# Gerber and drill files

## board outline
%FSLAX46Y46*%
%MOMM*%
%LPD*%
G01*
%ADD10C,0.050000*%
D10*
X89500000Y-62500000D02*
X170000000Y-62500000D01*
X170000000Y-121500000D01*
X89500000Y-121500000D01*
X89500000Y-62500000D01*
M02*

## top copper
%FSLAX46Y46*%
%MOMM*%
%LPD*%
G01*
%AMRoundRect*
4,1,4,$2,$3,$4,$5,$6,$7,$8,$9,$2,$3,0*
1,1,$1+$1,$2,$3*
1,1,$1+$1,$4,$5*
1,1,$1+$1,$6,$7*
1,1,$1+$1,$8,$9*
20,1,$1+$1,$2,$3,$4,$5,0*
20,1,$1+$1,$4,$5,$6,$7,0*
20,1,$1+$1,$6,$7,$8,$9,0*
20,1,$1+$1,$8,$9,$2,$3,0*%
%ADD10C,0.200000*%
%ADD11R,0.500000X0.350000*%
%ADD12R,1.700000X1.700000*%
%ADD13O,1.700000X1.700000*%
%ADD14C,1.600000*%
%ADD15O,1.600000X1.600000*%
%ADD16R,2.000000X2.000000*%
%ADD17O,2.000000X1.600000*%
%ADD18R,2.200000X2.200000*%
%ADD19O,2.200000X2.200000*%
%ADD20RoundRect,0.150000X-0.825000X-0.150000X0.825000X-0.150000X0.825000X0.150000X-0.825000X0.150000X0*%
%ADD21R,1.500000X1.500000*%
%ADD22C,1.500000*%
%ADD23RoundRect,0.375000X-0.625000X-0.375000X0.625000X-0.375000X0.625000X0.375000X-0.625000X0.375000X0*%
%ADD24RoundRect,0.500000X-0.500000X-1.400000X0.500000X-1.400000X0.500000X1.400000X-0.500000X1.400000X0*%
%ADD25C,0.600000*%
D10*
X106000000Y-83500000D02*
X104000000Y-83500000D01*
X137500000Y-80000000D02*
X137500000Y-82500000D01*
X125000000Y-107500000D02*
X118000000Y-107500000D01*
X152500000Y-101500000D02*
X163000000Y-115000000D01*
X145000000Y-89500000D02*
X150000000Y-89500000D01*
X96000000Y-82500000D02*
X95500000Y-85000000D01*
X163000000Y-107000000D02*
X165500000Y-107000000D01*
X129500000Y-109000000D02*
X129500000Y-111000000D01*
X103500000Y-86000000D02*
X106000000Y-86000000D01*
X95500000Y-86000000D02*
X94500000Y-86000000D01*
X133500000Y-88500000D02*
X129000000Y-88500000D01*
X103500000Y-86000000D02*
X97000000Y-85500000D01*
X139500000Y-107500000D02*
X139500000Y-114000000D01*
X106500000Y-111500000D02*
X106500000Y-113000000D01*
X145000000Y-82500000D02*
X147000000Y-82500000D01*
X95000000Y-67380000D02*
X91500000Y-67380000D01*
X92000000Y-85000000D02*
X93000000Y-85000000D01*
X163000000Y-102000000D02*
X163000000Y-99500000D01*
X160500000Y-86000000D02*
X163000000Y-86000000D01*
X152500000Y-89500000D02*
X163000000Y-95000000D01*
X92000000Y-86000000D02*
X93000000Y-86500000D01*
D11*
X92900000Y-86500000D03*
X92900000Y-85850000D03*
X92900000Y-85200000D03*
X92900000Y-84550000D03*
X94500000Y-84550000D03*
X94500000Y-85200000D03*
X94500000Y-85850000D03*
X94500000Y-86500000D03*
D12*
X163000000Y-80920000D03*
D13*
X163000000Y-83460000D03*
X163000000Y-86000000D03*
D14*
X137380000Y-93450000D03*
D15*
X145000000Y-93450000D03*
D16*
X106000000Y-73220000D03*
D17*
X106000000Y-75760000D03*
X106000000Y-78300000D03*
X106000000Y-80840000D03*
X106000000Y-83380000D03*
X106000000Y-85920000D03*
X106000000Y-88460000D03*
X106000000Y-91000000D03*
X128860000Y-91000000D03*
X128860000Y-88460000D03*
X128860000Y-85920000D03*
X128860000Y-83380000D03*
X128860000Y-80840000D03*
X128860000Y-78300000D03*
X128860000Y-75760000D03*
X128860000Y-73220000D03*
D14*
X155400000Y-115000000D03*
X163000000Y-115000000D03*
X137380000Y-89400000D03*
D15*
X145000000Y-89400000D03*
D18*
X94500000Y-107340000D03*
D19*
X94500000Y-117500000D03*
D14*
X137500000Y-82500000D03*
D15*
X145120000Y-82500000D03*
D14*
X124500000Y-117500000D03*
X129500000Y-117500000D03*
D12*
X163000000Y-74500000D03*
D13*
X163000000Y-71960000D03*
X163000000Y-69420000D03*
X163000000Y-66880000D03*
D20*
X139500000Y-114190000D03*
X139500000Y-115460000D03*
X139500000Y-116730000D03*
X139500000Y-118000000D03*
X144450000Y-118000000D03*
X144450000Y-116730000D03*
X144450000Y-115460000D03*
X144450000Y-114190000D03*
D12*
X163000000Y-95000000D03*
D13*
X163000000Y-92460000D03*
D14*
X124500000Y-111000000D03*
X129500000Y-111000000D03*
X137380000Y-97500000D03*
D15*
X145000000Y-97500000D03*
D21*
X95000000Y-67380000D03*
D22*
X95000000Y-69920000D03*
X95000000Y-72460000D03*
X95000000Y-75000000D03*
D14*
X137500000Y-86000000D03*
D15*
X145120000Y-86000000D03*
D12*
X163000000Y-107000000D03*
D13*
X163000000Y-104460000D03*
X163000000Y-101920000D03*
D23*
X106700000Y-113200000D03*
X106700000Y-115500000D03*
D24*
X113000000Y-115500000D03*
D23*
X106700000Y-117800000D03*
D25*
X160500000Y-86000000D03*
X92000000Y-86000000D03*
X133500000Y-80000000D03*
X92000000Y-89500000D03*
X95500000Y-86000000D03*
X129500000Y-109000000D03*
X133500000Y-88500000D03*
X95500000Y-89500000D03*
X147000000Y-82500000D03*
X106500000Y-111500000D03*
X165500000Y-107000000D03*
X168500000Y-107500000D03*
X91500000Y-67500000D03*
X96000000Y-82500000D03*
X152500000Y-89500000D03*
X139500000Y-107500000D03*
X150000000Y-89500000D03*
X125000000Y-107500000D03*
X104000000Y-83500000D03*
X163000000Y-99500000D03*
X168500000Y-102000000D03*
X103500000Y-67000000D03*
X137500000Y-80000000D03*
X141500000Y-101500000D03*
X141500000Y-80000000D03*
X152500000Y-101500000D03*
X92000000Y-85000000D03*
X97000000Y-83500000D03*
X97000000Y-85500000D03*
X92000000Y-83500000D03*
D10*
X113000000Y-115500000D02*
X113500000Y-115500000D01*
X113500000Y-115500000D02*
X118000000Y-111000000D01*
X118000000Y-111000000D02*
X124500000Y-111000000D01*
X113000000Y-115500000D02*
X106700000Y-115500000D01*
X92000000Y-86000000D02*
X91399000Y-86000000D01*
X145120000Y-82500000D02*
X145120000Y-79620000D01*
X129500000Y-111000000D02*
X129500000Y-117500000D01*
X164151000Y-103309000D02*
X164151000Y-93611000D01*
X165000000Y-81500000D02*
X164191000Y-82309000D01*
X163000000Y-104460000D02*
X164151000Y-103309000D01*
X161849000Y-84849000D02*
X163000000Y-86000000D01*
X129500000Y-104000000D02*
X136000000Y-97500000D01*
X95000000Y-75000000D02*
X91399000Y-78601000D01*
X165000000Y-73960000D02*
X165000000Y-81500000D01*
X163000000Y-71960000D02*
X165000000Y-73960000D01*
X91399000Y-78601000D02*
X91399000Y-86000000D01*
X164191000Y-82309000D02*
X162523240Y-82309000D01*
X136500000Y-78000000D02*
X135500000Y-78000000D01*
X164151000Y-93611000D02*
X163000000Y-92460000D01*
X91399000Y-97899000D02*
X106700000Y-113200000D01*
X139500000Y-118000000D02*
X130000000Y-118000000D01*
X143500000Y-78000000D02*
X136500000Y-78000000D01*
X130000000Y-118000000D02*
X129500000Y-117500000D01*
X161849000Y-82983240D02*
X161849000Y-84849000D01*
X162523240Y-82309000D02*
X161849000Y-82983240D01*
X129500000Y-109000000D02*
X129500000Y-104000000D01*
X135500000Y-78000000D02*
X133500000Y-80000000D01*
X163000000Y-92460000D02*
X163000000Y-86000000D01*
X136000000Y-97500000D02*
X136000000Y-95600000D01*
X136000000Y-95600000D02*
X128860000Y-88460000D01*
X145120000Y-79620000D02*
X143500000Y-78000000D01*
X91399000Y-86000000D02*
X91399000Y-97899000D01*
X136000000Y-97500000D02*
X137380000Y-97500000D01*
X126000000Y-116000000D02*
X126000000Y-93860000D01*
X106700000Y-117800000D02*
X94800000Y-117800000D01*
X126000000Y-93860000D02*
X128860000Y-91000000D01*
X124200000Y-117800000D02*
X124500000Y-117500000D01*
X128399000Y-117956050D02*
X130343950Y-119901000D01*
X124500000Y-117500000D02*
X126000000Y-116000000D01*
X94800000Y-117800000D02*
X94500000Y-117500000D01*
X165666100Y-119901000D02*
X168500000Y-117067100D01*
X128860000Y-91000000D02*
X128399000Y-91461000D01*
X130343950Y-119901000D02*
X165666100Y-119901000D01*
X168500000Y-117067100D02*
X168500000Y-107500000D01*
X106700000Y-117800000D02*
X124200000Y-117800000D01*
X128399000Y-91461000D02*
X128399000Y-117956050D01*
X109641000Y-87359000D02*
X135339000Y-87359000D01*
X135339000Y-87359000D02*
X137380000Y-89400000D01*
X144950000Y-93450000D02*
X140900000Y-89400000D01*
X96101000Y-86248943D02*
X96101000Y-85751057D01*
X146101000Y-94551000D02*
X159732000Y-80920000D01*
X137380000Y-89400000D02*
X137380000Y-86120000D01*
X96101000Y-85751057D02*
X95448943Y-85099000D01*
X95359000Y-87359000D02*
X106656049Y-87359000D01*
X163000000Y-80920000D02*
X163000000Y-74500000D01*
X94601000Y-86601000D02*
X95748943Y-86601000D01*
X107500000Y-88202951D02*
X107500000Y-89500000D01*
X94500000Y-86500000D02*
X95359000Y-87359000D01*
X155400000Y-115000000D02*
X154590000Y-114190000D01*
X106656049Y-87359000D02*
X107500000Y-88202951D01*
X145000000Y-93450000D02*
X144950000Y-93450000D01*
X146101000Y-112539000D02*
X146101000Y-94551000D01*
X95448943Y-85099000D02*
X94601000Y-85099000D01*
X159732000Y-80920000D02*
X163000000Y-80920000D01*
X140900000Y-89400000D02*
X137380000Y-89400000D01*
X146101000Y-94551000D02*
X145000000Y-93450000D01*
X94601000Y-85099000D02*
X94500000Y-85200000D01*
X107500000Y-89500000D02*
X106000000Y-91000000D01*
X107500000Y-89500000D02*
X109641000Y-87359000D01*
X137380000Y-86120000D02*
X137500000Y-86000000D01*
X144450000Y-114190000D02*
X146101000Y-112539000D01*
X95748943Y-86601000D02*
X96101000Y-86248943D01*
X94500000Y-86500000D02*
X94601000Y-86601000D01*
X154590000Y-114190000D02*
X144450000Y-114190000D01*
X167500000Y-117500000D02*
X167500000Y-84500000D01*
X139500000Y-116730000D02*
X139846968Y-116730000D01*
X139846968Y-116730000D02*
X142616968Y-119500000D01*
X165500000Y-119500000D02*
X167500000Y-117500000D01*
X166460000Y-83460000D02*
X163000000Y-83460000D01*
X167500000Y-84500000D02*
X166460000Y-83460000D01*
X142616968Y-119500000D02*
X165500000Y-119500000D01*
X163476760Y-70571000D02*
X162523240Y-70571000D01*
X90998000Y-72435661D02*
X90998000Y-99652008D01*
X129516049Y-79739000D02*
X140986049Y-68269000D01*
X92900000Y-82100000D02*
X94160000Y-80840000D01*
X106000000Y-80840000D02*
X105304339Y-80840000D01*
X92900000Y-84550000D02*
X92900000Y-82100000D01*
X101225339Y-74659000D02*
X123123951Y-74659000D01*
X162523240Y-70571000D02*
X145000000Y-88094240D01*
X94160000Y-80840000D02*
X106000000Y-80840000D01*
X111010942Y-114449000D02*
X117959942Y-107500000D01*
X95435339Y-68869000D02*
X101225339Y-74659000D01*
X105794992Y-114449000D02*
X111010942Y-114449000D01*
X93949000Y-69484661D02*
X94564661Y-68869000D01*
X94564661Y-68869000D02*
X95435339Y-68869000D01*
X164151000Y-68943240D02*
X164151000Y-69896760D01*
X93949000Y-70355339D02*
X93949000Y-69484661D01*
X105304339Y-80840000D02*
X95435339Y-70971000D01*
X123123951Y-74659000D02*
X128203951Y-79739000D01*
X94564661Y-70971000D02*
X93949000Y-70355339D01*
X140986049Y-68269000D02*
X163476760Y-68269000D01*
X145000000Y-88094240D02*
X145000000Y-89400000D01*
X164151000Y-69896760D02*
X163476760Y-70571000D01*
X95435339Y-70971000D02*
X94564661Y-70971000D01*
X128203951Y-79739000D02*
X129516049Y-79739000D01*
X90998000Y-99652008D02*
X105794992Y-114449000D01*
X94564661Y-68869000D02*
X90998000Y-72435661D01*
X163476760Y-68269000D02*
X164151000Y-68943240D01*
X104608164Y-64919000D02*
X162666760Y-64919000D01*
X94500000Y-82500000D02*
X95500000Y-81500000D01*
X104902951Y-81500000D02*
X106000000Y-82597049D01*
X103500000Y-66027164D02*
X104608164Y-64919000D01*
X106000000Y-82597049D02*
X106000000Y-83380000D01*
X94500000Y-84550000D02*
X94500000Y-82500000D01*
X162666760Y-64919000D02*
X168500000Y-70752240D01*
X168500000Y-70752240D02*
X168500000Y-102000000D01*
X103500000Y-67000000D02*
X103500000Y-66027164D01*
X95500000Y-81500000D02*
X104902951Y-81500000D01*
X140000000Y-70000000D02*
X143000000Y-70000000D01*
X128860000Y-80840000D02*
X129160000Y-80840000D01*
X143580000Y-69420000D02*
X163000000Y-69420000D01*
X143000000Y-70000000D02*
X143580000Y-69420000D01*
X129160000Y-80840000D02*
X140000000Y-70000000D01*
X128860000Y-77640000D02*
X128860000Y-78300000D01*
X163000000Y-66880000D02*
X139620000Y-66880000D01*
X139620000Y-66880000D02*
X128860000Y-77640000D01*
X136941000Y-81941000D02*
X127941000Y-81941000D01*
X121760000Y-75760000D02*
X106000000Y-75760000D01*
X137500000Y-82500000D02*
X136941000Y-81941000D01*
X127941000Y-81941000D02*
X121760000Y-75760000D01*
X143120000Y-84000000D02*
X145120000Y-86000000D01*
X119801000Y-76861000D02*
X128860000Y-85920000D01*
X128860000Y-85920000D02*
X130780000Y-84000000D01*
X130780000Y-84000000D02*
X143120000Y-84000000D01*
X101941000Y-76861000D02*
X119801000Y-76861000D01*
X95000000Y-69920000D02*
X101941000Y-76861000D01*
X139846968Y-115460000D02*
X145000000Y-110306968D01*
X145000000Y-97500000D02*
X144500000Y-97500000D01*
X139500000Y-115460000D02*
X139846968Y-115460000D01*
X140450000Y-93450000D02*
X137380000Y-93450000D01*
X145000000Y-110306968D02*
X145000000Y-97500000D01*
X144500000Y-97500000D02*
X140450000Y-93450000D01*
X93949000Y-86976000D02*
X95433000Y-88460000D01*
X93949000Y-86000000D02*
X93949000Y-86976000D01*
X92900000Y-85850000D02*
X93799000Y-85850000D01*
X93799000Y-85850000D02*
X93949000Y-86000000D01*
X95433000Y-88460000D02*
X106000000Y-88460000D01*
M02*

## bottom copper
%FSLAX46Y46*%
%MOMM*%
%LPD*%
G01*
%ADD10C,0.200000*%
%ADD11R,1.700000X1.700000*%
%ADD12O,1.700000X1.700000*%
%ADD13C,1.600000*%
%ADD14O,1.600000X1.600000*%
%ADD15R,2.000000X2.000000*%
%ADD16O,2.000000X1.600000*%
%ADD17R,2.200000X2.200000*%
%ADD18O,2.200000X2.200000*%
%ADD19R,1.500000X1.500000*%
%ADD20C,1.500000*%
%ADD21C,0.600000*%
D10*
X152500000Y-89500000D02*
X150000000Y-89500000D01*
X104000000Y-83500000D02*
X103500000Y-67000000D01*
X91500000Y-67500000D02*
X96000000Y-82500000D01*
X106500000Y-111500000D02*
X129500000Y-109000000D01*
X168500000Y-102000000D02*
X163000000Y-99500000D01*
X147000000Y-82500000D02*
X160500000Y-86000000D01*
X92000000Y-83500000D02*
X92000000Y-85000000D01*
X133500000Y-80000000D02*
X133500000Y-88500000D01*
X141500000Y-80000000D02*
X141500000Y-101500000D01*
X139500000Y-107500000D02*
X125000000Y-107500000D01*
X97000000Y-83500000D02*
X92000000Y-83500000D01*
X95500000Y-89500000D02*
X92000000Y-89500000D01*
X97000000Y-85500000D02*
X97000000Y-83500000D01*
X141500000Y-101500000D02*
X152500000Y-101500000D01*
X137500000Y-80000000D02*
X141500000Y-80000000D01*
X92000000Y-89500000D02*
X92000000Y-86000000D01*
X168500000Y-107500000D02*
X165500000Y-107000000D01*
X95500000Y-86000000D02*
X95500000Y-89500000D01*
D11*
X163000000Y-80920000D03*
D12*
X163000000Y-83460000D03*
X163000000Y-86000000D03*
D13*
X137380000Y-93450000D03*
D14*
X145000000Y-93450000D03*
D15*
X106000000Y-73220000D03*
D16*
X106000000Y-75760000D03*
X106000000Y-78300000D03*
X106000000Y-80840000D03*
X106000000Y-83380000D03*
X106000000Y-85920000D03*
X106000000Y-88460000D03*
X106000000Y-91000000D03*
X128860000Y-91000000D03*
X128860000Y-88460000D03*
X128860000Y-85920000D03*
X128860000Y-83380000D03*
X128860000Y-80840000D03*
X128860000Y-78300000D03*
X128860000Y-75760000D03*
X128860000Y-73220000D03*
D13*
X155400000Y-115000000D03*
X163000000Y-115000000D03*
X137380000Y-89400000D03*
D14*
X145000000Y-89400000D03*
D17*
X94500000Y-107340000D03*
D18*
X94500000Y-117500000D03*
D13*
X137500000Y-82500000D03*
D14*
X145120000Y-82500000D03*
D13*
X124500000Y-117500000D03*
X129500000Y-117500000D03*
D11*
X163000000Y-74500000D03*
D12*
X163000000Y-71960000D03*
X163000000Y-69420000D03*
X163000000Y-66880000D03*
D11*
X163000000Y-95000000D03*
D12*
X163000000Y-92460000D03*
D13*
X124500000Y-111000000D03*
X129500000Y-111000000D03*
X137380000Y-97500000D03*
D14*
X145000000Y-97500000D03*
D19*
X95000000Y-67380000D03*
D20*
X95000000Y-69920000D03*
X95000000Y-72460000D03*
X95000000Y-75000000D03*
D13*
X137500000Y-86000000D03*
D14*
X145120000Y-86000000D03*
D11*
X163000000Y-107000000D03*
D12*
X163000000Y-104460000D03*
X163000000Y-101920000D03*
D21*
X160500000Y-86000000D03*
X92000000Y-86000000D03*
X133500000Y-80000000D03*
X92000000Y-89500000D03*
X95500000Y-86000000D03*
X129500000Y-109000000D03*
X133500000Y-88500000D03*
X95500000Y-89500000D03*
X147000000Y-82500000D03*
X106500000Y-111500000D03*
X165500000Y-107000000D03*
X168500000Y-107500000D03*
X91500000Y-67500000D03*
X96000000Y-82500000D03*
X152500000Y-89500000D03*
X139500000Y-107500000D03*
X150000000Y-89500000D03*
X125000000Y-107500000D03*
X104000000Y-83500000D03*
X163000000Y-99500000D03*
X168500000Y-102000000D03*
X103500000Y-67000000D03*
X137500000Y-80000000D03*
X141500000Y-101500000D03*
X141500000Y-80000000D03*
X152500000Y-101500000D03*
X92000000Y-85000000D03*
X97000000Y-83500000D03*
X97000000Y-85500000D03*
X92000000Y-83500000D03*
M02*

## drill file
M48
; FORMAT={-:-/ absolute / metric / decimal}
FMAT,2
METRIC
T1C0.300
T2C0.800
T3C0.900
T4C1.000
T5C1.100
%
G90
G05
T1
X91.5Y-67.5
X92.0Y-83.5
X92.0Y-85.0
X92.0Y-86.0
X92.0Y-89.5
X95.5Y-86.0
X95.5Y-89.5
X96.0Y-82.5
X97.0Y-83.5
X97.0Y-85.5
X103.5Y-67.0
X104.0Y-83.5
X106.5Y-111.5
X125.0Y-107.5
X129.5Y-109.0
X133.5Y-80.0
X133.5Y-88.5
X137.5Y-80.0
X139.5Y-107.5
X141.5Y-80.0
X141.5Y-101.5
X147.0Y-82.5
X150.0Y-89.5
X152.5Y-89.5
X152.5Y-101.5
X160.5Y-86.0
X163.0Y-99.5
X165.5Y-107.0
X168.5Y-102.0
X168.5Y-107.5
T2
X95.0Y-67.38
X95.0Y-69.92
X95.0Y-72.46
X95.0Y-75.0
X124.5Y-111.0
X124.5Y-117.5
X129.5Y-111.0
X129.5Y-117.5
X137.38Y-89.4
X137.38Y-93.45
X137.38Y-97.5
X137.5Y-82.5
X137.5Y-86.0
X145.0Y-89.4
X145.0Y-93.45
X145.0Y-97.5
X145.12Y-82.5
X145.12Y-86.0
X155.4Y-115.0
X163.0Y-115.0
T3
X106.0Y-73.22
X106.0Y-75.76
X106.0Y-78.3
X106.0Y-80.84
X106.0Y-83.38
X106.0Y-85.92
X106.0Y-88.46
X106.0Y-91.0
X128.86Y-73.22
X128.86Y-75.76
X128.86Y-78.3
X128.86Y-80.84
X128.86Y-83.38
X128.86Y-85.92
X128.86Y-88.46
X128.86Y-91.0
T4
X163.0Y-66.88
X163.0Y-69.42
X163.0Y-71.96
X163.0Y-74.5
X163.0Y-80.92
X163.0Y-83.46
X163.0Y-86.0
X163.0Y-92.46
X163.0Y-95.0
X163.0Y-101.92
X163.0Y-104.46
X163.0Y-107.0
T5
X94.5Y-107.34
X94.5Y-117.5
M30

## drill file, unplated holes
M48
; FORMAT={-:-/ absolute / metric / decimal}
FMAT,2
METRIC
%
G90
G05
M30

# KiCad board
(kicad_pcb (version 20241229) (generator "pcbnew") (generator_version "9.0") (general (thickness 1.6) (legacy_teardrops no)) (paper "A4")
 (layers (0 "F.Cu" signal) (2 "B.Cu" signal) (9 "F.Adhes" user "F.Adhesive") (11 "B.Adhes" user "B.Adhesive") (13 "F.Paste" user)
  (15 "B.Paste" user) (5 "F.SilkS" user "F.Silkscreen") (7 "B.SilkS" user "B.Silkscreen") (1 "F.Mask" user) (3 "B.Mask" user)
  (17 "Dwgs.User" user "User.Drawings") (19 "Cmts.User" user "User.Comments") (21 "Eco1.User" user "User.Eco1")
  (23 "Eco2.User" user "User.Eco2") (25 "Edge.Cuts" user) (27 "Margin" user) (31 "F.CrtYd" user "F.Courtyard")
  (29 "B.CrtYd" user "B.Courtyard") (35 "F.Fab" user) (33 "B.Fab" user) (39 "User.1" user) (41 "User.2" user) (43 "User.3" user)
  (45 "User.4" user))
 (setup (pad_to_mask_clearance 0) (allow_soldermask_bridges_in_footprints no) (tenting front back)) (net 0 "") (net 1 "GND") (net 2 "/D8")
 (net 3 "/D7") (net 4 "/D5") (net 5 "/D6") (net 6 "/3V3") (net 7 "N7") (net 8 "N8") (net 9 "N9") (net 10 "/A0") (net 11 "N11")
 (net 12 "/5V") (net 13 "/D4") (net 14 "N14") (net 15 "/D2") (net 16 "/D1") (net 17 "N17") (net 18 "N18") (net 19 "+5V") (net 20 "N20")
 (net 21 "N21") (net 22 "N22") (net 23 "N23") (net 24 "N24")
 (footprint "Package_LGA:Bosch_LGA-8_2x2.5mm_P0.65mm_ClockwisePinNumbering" (layer "F.Cu") (at 93.7 85.525 90)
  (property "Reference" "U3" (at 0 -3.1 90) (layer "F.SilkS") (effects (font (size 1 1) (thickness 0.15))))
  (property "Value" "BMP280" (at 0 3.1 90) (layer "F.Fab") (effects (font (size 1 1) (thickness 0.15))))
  (pad "1" smd rect (at -0.975 -0.8 180) (size 0.5 0.35) (layers "F.Cu" "F.Mask" "F.Paste") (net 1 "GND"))
  (pad "2" smd rect (at -0.325 -0.8 180) (size 0.5 0.35) (layers "F.Cu" "F.Mask" "F.Paste") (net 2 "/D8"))
  (pad "3" smd rect (at 0.325 -0.8 180) (size 0.5 0.35) (layers "F.Cu" "F.Mask" "F.Paste") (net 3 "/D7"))
  (pad "4" smd rect (at 0.975 -0.8 180) (size 0.5 0.35) (layers "F.Cu" "F.Mask" "F.Paste") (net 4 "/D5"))
  (pad "5" smd rect (at 0.975 0.8 180) (size 0.5 0.35) (layers "F.Cu" "F.Mask" "F.Paste") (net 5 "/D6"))
  (pad "6" smd rect (at 0.325 0.8 180) (size 0.5 0.35) (layers "F.Cu" "F.Mask" "F.Paste") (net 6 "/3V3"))
  (pad "7" smd rect (at -0.325 0.8 180) (size 0.5 0.35) (layers "F.Cu" "F.Mask" "F.Paste") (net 1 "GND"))
  (pad "8" smd rect (at -0.975 0.8 180) (size 0.5 0.35) (layers "F.Cu" "F.Mask" "F.Paste") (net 6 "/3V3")))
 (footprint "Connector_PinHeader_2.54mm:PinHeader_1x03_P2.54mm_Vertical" (layer "F.Cu") (at 163 80.92)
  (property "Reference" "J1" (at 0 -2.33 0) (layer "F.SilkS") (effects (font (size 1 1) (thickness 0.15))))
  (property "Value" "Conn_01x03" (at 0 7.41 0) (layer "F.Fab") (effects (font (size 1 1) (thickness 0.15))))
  (pad "1" thru_hole rect (at 0 0) (size 1.7 1.7) (drill 1) (layers "*.Cu" "*.Mask") (remove_unused_layers no) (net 6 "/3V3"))
  (pad "2" thru_hole oval (at 0 2.54) (size 1.7 1.7) (drill 1) (layers "*.Cu" "*.Mask") (remove_unused_layers no) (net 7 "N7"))
  (pad "3" thru_hole oval (at 0 5.08) (size 1.7 1.7) (drill 1) (layers "*.Cu" "*.Mask") (remove_unused_layers no) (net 1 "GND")))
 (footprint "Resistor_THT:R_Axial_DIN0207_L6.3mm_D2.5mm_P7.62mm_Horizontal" (layer "F.Cu") (at 137.38 93.45)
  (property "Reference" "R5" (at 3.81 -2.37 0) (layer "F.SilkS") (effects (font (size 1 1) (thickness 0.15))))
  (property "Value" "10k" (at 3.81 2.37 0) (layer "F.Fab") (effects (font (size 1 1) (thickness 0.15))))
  (pad "1" thru_hole circle (at 0 0) (size 1.6 1.6) (drill 0.8) (layers "*.Cu" "*.Mask") (remove_unused_layers no) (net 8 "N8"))
  (pad "2" thru_hole oval (at 7.62 0) (size 1.6 1.6) (drill 0.8) (layers "*.Cu" "*.Mask") (remove_unused_layers no) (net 6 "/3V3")))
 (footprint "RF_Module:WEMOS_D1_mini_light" (layer "F.Cu") (at 106 73.22)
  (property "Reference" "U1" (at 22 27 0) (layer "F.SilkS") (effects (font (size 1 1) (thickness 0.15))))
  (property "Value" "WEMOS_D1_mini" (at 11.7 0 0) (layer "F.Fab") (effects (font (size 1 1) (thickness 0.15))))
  (pad "1" thru_hole rect (at 0 0) (size 2 2) (drill 0.9) (layers "*.Cu" "*.Mask") (remove_unused_layers no) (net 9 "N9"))
  (pad "2" thru_hole oval (at 0 2.54) (size 2 1.6) (drill 0.9) (layers "*.Cu" "*.Mask") (remove_unused_layers no) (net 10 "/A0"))
  (pad "3" thru_hole oval (at 0 5.08) (size 2 1.6) (drill 0.9) (layers "*.Cu" "*.Mask") (remove_unused_layers no) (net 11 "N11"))
  (pad "4" thru_hole oval (at 0 7.62) (size 2 1.6) (drill 0.9) (layers "*.Cu" "*.Mask") (remove_unused_layers no) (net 4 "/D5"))
  (pad "5" thru_hole oval (at 0 10.16) (size 2 1.6) (drill 0.9) (layers "*.Cu" "*.Mask") (remove_unused_layers no) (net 5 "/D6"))
  (pad "6" thru_hole oval (at 0 12.7) (size 2 1.6) (drill 0.9) (layers "*.Cu" "*.Mask") (remove_unused_layers no) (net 3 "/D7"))
  (pad "7" thru_hole oval (at 0 15.24) (size 2 1.6) (drill 0.9) (layers "*.Cu" "*.Mask") (remove_unused_layers no) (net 2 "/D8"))
  (pad "8" thru_hole oval (at 0 17.78) (size 2 1.6) (drill 0.9) (layers "*.Cu" "*.Mask") (remove_unused_layers no) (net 6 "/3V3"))
  (pad "9" thru_hole oval (at 22.86 17.78) (size 2 1.6) (drill 0.9) (layers "*.Cu" "*.Mask") (remove_unused_layers no) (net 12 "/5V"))
  (pad "10" thru_hole oval (at 22.86 15.24) (size 2 1.6) (drill 0.9) (layers "*.Cu" "*.Mask") (remove_unused_layers no) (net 1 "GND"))
  (pad "11" thru_hole oval (at 22.86 12.7) (size 2 1.6) (drill 0.9) (layers "*.Cu" "*.Mask") (remove_unused_layers no) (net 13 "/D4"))
  (pad "12" thru_hole oval (at 22.86 10.16) (size 2 1.6) (drill 0.9) (layers "*.Cu" "*.Mask") (remove_unused_layers no) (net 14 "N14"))
  (pad "13" thru_hole oval (at 22.86 7.62) (size 2 1.6) (drill 0.9) (layers "*.Cu" "*.Mask") (remove_unused_layers no) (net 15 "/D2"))
  (pad "14" thru_hole oval (at 22.86 5.08) (size 2 1.6) (drill 0.9) (layers "*.Cu" "*.Mask") (remove_unused_layers no) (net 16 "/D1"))
  (pad "15" thru_hole oval (at 22.86 2.54) (size 2 1.6) (drill 0.9) (layers "*.Cu" "*.Mask") (remove_unused_layers no) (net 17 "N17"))
  (pad "16" thru_hole oval (at 22.86 0) (size 2 1.6) (drill 0.9) (layers "*.Cu" "*.Mask") (remove_unused_layers no) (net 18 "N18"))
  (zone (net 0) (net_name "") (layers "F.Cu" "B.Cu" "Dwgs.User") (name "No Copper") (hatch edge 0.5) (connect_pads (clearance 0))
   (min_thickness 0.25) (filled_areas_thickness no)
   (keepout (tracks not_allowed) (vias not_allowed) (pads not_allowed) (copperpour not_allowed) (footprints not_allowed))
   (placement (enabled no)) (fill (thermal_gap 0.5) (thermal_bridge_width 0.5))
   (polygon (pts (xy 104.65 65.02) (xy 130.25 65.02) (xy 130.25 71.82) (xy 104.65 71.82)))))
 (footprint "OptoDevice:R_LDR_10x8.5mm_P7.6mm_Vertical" (layer "F.Cu") (at 155.4 115)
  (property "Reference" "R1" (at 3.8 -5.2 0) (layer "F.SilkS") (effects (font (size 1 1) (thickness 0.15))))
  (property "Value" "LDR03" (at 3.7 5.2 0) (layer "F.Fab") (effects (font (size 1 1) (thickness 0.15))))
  (pad "1" thru_hole circle (at 0 0) (size 1.6 1.6) (drill 0.8) (layers "*.Cu" "*.Mask") (remove_unused_layers no) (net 6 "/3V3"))
  (pad "2" thru_hole circle (at 7.6 0) (size 1.6 1.6) (drill 0.8) (layers "*.Cu" "*.Mask") (remove_unused_layers no) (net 10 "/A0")))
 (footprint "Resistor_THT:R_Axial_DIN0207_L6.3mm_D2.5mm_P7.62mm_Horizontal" (layer "F.Cu") (at 137.38 89.4)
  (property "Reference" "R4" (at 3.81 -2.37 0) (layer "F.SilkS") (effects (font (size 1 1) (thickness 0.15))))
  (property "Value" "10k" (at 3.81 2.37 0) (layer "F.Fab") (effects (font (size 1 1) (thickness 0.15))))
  (pad "1" thru_hole circle (at 0 0) (size 1.6 1.6) (drill 0.8) (layers "*.Cu" "*.Mask") (remove_unused_layers no) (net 6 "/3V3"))
  (pad "2" thru_hole oval (at 7.62 0) (size 1.6 1.6) (drill 0.8) (layers "*.Cu" "*.Mask") (remove_unused_layers no) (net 4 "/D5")))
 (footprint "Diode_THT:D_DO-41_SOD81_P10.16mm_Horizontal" (layer "F.Cu") (at 94.5 107.34 -90)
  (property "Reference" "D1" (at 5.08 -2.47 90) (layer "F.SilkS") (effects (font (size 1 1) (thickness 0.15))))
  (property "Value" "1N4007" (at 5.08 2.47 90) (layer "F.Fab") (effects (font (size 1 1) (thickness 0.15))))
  (pad "1" thru_hole rect (at 0 0 270) (size 2.2 2.2) (drill 1.1) (layers "*.Cu" "*.Mask") (remove_unused_layers no) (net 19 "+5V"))
  (pad "2" thru_hole oval (at 10.16 0 270) (size 2.2 2.2) (drill 1.1) (layers "*.Cu" "*.Mask") (remove_unused_layers no) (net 12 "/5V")))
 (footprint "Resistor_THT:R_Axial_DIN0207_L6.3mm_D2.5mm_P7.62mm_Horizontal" (layer "F.Cu") (at 137.5 82.5)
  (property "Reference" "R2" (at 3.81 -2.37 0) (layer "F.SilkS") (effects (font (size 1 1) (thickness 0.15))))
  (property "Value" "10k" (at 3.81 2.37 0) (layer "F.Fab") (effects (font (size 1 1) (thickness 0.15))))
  (pad "1" thru_hole circle (at 0 0) (size 1.6 1.6) (drill 0.8) (layers "*.Cu" "*.Mask") (remove_unused_layers no) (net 10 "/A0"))
  (pad "2" thru_hole oval (at 7.62 0) (size 1.6 1.6) (drill 0.8) (layers "*.Cu" "*.Mask") (remove_unused_layers no) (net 1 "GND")))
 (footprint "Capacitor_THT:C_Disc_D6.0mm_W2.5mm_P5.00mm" (layer "F.Cu") (at 124.5 117.5)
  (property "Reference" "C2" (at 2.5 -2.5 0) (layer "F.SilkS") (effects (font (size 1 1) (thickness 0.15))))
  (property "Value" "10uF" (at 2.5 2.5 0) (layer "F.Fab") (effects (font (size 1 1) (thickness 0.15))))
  (pad "1" thru_hole circle (at 0 0) (size 1.6 1.6) (drill 0.8) (layers "*.Cu" "*.Mask") (remove_unused_layers no) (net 12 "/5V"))
  (pad "2" thru_hole circle (at 5 0) (size 1.6 1.6) (drill 0.8) (layers "*.Cu" "*.Mask") (remove_unused_layers no) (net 1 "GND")))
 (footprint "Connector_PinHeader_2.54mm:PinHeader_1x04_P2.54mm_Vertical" (layer "F.Cu") (at 163 74.5 180)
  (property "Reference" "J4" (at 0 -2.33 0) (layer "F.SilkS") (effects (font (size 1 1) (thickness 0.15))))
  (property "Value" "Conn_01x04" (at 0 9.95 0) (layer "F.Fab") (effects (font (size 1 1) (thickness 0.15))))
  (pad "1" thru_hole rect (at 0 0 180) (size 1.7 1.7) (drill 1) (layers "*.Cu" "*.Mask") (remove_unused_layers no) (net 6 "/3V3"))
  (pad "2" thru_hole oval (at 0 2.54 180) (size 1.7 1.7) (drill 1) (layers "*.Cu" "*.Mask") (remove_unused_layers no) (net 1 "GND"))
  (pad "3" thru_hole oval (at 0 5.08 180) (size 1.7 1.7) (drill 1) (layers "*.Cu" "*.Mask") (remove_unused_layers no) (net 15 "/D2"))
  (pad "4" thru_hole oval (at 0 7.62 180) (size 1.7 1.7) (drill 1) (layers "*.Cu" "*.Mask") (remove_unused_layers no) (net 16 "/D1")))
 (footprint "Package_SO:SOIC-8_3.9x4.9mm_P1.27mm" (layer "F.Cu") (at 141.975 116.095)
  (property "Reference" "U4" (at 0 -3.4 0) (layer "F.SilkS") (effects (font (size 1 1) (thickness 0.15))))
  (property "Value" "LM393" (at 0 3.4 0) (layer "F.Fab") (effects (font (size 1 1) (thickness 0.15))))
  (pad "1" smd roundrect (at -2.475 -1.905) (size 1.95 0.6) (layers "F.Cu" "F.Mask" "F.Paste") (roundrect_rratio 0.25) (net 4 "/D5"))
  (pad "2" smd roundrect (at -2.475 -0.635) (size 1.95 0.6) (layers "F.Cu" "F.Mask" "F.Paste") (roundrect_rratio 0.25) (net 8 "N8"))
  (pad "3" smd roundrect (at -2.475 0.635) (size 1.95 0.6) (layers "F.Cu" "F.Mask" "F.Paste") (roundrect_rratio 0.25) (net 7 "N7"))
  (pad "4" smd roundrect (at -2.475 1.905) (size 1.95 0.6) (layers "F.Cu" "F.Mask" "F.Paste") (roundrect_rratio 0.25) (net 1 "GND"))
  (pad "5" smd roundrect (at 2.475 1.905) (size 1.95 0.6) (layers "F.Cu" "F.Mask" "F.Paste") (roundrect_rratio 0.25) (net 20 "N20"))
  (pad "6" smd roundrect (at 2.475 0.635) (size 1.95 0.6) (layers "F.Cu" "F.Mask" "F.Paste") (roundrect_rratio 0.25) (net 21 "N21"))
  (pad "7" smd roundrect (at 2.475 -0.635) (size 1.95 0.6) (layers "F.Cu" "F.Mask" "F.Paste") (roundrect_rratio 0.25) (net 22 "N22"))
  (pad "8" smd roundrect (at 2.475 -1.905) (size 1.95 0.6) (layers "F.Cu" "F.Mask" "F.Paste") (roundrect_rratio 0.25) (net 6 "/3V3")))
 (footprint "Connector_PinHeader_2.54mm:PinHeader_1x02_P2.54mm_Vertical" (layer "F.Cu") (at 163 95 180)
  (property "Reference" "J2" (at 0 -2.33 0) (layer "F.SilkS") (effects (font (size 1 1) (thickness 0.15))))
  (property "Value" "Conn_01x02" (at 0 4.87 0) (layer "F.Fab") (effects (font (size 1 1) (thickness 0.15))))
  (pad "1" thru_hole rect (at 0 0 180) (size 1.7 1.7) (drill 1) (layers "*.Cu" "*.Mask") (remove_unused_layers no) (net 4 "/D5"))
  (pad "2" thru_hole oval (at 0 2.54 180) (size 1.7 1.7) (drill 1) (layers "*.Cu" "*.Mask") (remove_unused_layers no) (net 1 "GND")))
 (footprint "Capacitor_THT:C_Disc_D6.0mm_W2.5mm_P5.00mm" (layer "F.Cu") (at 124.5 111)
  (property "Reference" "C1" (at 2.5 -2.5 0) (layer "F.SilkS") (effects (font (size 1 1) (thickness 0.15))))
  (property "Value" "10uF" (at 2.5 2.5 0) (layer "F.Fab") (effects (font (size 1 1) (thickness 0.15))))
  (pad "1" thru_hole circle (at 0 0) (size 1.6 1.6) (drill 0.8) (layers "*.Cu" "*.Mask") (remove_unused_layers no) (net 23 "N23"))
  (pad "2" thru_hole circle (at 5 0) (size 1.6 1.6) (drill 0.8) (layers "*.Cu" "*.Mask") (remove_unused_layers no) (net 1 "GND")))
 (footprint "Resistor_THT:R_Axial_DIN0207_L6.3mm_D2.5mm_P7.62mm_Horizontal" (layer "F.Cu") (at 137.38 97.5)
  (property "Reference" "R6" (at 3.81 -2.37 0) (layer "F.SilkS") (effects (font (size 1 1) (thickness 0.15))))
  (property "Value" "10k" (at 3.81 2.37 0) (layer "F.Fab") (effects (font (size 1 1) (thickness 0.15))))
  (pad "1" thru_hole circle (at 0 0) (size 1.6 1.6) (drill 0.8) (layers "*.Cu" "*.Mask") (remove_unused_layers no) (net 1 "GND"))
  (pad "2" thru_hole oval (at 7.62 0) (size 1.6 1.6) (drill 0.8) (layers "*.Cu" "*.Mask") (remove_unused_layers no) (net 8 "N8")))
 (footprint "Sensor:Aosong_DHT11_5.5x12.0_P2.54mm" (layer "F.Cu") (at 95 67.38)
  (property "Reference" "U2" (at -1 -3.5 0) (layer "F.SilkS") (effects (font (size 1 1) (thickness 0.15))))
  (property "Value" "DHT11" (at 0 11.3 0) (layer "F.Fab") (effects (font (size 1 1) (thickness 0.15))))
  (pad "1" thru_hole rect (at 0 0) (size 1.5 1.5) (drill 0.8) (layers "*.Cu" "*.Mask") (remove_unused_layers no) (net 6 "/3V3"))
  (pad "2" thru_hole circle (at 0 2.54) (size 1.5 1.5) (drill 0.8) (layers "*.Cu" "*.Mask") (remove_unused_layers no) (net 13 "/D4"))
  (pad "3" thru_hole circle (at 0 5.08) (size 1.5 1.5) (drill 0.8) (layers "*.Cu" "*.Mask") (remove_unused_layers no) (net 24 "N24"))
  (pad "4" thru_hole circle (at 0 7.62) (size 1.5 1.5) (drill 0.8) (layers "*.Cu" "*.Mask") (remove_unused_layers no) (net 1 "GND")))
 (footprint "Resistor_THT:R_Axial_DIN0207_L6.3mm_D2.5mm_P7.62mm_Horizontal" (layer "F.Cu") (at 137.5 86)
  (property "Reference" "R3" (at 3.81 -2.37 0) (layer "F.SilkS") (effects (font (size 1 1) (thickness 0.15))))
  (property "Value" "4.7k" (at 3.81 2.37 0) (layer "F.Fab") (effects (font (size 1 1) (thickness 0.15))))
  (pad "1" thru_hole circle (at 0 0) (size 1.6 1.6) (drill 0.8) (layers "*.Cu" "*.Mask") (remove_unused_layers no) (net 6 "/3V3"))
  (pad "2" thru_hole oval (at 7.62 0) (size 1.6 1.6) (drill 0.8) (layers "*.Cu" "*.Mask") (remove_unused_layers no) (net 13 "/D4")))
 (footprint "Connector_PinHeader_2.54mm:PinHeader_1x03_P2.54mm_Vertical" (layer "F.Cu") (at 163 107 180)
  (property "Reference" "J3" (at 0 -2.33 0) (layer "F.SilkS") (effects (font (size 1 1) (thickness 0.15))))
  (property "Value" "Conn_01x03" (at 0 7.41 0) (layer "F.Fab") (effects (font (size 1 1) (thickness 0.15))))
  (pad "1" thru_hole rect (at 0 0 180) (size 1.7 1.7) (drill 1) (layers "*.Cu" "*.Mask") (remove_unused_layers no) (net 12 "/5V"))
  (pad "2" thru_hole oval (at 0 2.54 180) (size 1.7 1.7) (drill 1) (layers "*.Cu" "*.Mask") (remove_unused_layers no) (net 1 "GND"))
  (pad "3" thru_hole oval (at 0 5.08 180) (size 1.7 1.7) (drill 1) (layers "*.Cu" "*.Mask") (remove_unused_layers no) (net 5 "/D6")))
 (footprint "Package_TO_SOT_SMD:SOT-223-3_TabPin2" (layer "F.Cu") (at 109.85 115.5)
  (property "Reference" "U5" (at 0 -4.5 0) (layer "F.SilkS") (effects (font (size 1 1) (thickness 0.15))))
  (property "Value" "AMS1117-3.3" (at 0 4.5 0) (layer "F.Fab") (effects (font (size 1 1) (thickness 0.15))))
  (pad "1" smd roundrect (at -3.15 -2.3) (size 2 1.5) (layers "F.Cu" "F.Mask" "F.Paste") (roundrect_rratio 0.25) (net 1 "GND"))
  (pad "2" smd roundrect (at -3.15 0) (size 2 1.5) (layers "F.Cu" "F.Mask" "F.Paste") (roundrect_rratio 0.25) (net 23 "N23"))
  (pad "2" smd roundrect (at 3.15 0) (size 2 3.8) (layers "F.Cu" "F.Mask" "F.Paste") (roundrect_rratio 0.25) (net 23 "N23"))
  (pad "3" smd roundrect (at -3.15 2.3) (size 2 1.5) (layers "F.Cu" "F.Mask" "F.Paste") (roundrect_rratio 0.25) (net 12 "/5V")))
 (gr_line (start 106 83.5) (end 104 83.5) (stroke (width 0.2) (type default)) (layer "F.Cu") (net 5))
 (gr_line (start 137.5 80) (end 137.5 82.5) (stroke (width 0.2) (type default)) (layer "F.Cu") (net 10))
 (gr_line (start 125 107.5) (end 118 107.5) (stroke (width 0.2) (type default)) (layer "F.Cu") (net 4))
 (gr_line (start 152.5 101.5) (end 163 115) (stroke (width 0.2) (type default)) (layer "F.Cu") (net 10))
 (gr_line (start 145 89.5) (end 150 89.5) (stroke (width 0.2) (type default)) (layer "F.Cu") (net 4))
 (gr_line (start 96 82.5) (end 95.5 85) (stroke (width 0.2) (type default)) (layer "F.Cu") (net 6))
 (gr_line (start 163 107) (end 165.5 107) (stroke (width 0.2) (type default)) (layer "F.Cu") (net 12))
 (gr_line (start 129.5 109) (end 129.5 111) (stroke (width 0.2) (type default)) (layer "F.Cu") (net 1))
 (gr_line (start 103.5 86) (end 106 86) (stroke (width 0.2) (type default)) (layer "F.Cu") (net 3))
 (gr_line (start 95.5 86) (end 94.5 86) (stroke (width 0.2) (type default)) (layer "F.Cu") (net 1))
 (gr_line (start 133.5 88.5) (end 129 88.5) (stroke (width 0.2) (type default)) (layer "F.Cu") (net 1))
 (gr_line (start 103.5 86) (end 97 85.5) (stroke (width 0.2) (type default)) (layer "F.Cu") (net 3))
 (gr_line (start 139.5 107.5) (end 139.5 114) (stroke (width 0.2) (type default)) (layer "F.Cu") (net 4))
 (gr_line (start 106.5 111.5) (end 106.5 113) (stroke (width 0.2) (type default)) (layer "F.Cu") (net 1))
 (gr_line (start 145 82.5) (end 147 82.5) (stroke (width 0.2) (type default)) (layer "F.Cu") (net 1))
 (gr_line (start 95 67.38) (end 91.5 67.38) (stroke (width 0.2) (type default)) (layer "F.Cu") (net 6))
 (gr_line (start 92 85) (end 93 85) (stroke (width 0.2) (type default)) (layer "F.Cu") (net 3))
 (gr_line (start 163 102) (end 163 99.5) (stroke (width 0.2) (type default)) (layer "F.Cu") (net 5))
 (gr_line (start 160.5 86) (end 163 86) (stroke (width 0.2) (type default)) (layer "F.Cu") (net 1))
 (gr_line (start 152.5 89.5) (end 163 95) (stroke (width 0.2) (type default)) (layer "F.Cu") (net 4))
 (gr_line (start 92 86) (end 93 86.5) (stroke (width 0.2) (type default)) (layer "F.Cu") (net 1))
 (gr_line (start 152.5 89.5) (end 150 89.5) (stroke (width 0.2) (type default)) (layer "B.Cu") (net 4))
 (gr_line (start 104 83.5) (end 103.5 67) (stroke (width 0.2) (type default)) (layer "B.Cu") (net 5))
 (gr_line (start 91.5 67.5) (end 96 82.5) (stroke (width 0.2) (type default)) (layer "B.Cu") (net 6))
 (gr_line (start 106.5 111.5) (end 129.5 109) (stroke (width 0.2) (type default)) (layer "B.Cu") (net 1))
 (gr_line (start 168.5 102) (end 163 99.5) (stroke (width 0.2) (type default)) (layer "B.Cu") (net 5))
 (gr_line (start 147 82.5) (end 160.5 86) (stroke (width 0.2) (type default)) (layer "B.Cu") (net 1))
 (gr_line (start 92 83.5) (end 92 85) (stroke (width 0.2) (type default)) (layer "B.Cu") (net 3))
 (gr_line (start 133.5 80) (end 133.5 88.5) (stroke (width 0.2) (type default)) (layer "B.Cu") (net 1))
 (gr_line (start 141.5 80) (end 141.5 101.5) (stroke (width 0.2) (type default)) (layer "B.Cu") (net 10))
 (gr_line (start 139.5 107.5) (end 125 107.5) (stroke (width 0.2) (type default)) (layer "B.Cu") (net 4))
 (gr_line (start 97 83.5) (end 92 83.5) (stroke (width 0.2) (type default)) (layer "B.Cu") (net 3))
 (gr_line (start 95.5 89.5) (end 92 89.5) (stroke (width 0.2) (type default)) (layer "B.Cu") (net 1))
 (gr_line (start 97 85.5) (end 97 83.5) (stroke (width 0.2) (type default)) (layer "B.Cu") (net 3))
 (gr_line (start 141.5 101.5) (end 152.5 101.5) (stroke (width 0.2) (type default)) (layer "B.Cu") (net 10))
 (gr_line (start 137.5 80) (end 141.5 80) (stroke (width 0.2) (type default)) (layer "B.Cu") (net 10))
 (gr_line (start 92 89.5) (end 92 86) (stroke (width 0.2) (type default)) (layer "B.Cu") (net 1))
 (gr_line (start 168.5 107.5) (end 165.5 107) (stroke (width 0.2) (type default)) (layer "B.Cu") (net 12))
 (gr_line (start 95.5 86) (end 95.5 89.5) (stroke (width 0.2) (type default)) (layer "B.Cu") (net 1))
 (gr_rect (start 89.5 62.5) (end 170 121.5) (stroke (width 0.05) (type default)) (fill no) (layer "Edge.Cuts"))
 (segment (start 113 115.5) (end 113.5 115.5) (width 0.2) (layer "F.Cu") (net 23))
 (segment (start 113.5 115.5) (end 118 111) (width 0.2) (layer "F.Cu") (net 23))
 (segment (start 118 111) (end 124.5 111) (width 0.2) (layer "F.Cu") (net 23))
 (segment (start 113 115.5) (end 106.7 115.5) (width 0.2) (layer "F.Cu") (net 23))
 (segment (start 92 86) (end 91.399 86) (width 0.2) (layer "F.Cu") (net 1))
 (segment (start 145.12 82.5) (end 145.12 79.62) (width 0.2) (layer "F.Cu") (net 1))
 (segment (start 129.5 111) (end 129.5 117.5) (width 0.2) (layer "F.Cu") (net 1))
 (segment (start 164.151 103.309) (end 164.151 93.611) (width 0.2) (layer "F.Cu") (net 1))
 (segment (start 165 81.5) (end 164.191 82.309) (width 0.2) (layer "F.Cu") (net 1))
 (segment (start 163 104.46) (end 164.151 103.309) (width 0.2) (layer "F.Cu") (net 1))
 (segment (start 161.849 84.849) (end 163 86) (width 0.2) (layer "F.Cu") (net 1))
 (segment (start 129.5 104) (end 136 97.5) (width 0.2) (layer "F.Cu") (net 1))
 (segment (start 95 75) (end 91.399 78.601) (width 0.2) (layer "F.Cu") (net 1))
 (segment (start 165 73.96) (end 165 81.5) (width 0.2) (layer "F.Cu") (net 1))
 (segment (start 163 71.96) (end 165 73.96) (width 0.2) (layer "F.Cu") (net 1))
 (segment (start 91.399 78.601) (end 91.399 86) (width 0.2) (layer "F.Cu") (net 1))
 (segment (start 164.191 82.309) (end 162.52324 82.309) (width 0.2) (layer "F.Cu") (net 1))
 (segment (start 136.5 78) (end 135.5 78) (width 0.2) (layer "F.Cu") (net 1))
 (segment (start 164.151 93.611) (end 163 92.46) (width 0.2) (layer "F.Cu") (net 1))
 (segment (start 91.399 97.899) (end 106.7 113.2) (width 0.2) (layer "F.Cu") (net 1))
 (segment (start 139.5 118) (end 130 118) (width 0.2) (layer "F.Cu") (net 1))
 (segment (start 143.5 78) (end 136.5 78) (width 0.2) (layer "F.Cu") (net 1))
 (segment (start 130 118) (end 129.5 117.5) (width 0.2) (layer "F.Cu") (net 1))
 (segment (start 161.849 82.98324) (end 161.849 84.849) (width 0.2) (layer "F.Cu") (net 1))
 (segment (start 162.52324 82.309) (end 161.849 82.98324) (width 0.2) (layer "F.Cu") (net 1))
 (segment (start 129.5 109) (end 129.5 104) (width 0.2) (layer "F.Cu") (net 1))
 (segment (start 135.5 78) (end 133.5 80) (width 0.2) (layer "F.Cu") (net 1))
 (segment (start 163 92.46) (end 163 86) (width 0.2) (layer "F.Cu") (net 1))
 (segment (start 136 97.5) (end 136 95.6) (width 0.2) (layer "F.Cu") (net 1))
 (segment (start 136 95.6) (end 128.86 88.46) (width 0.2) (layer "F.Cu") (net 1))
 (segment (start 145.12 79.62) (end 143.5 78) (width 0.2) (layer "F.Cu") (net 1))
 (segment (start 91.399 86) (end 91.399 97.899) (width 0.2) (layer "F.Cu") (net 1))
 (segment (start 136 97.5) (end 137.38 97.5) (width 0.2) (layer "F.Cu") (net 1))
 (via (at 160.5 86) (size 0.6) (drill 0.3) (layers "F.Cu" "B.Cu") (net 1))
 (via (at 92 86) (size 0.6) (drill 0.3) (layers "F.Cu" "B.Cu") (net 1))
 (via (at 133.5 80) (size 0.6) (drill 0.3) (layers "F.Cu" "B.Cu") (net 1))
 (via (at 92 89.5) (size 0.6) (drill 0.3) (layers "F.Cu" "B.Cu") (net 1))
 (via (at 95.5 86) (size 0.6) (drill 0.3) (layers "F.Cu" "B.Cu") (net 1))
 (via (at 129.5 109) (size 0.6) (drill 0.3) (layers "F.Cu" "B.Cu") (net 1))
 (via (at 133.5 88.5) (size 0.6) (drill 0.3) (layers "F.Cu" "B.Cu") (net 1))
 (via (at 95.5 89.5) (size 0.6) (drill 0.3) (layers "F.Cu" "B.Cu") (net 1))
 (via (at 147 82.5) (size 0.6) (drill 0.3) (layers "F.Cu" "B.Cu") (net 1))
 (via (at 106.5 111.5) (size 0.6) (drill 0.3) (layers "F.Cu" "B.Cu") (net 1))
 (segment (start 126 116) (end 126 93.86) (width 0.2) (layer "F.Cu") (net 12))
 (segment (start 106.7 117.8) (end 94.8 117.8) (width 0.2) (layer "F.Cu") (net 12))
 (segment (start 126 93.86) (end 128.86 91) (width 0.2) (layer "F.Cu") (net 12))
 (segment (start 124.2 117.8) (end 124.5 117.5) (width 0.2) (layer "F.Cu") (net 12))
 (segment (start 128.399 117.95605) (end 130.34395 119.901) (width 0.2) (layer "F.Cu") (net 12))
 (segment (start 124.5 117.5) (end 126 116) (width 0.2) (layer "F.Cu") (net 12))
 (segment (start 94.8 117.8) (end 94.5 117.5) (width 0.2) (layer "F.Cu") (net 12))
 (segment (start 165.6661 119.901) (end 168.5 117.0671) (width 0.2) (layer "F.Cu") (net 12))
 (segment (start 128.86 91) (end 128.399 91.461) (width 0.2) (layer "F.Cu") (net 12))
 (segment (start 130.34395 119.901) (end 165.6661 119.901) (width 0.2) (layer "F.Cu") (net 12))
 (segment (start 168.5 117.0671) (end 168.5 107.5) (width 0.2) (layer "F.Cu") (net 12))
 (segment (start 106.7 117.8) (end 124.2 117.8) (width 0.2) (layer "F.Cu") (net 12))
 (segment (start 128.399 91.461) (end 128.399 117.95605) (width 0.2) (layer "F.Cu") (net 12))
 (via (at 165.5 107) (size 0.6) (drill 0.3) (layers "F.Cu" "B.Cu") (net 12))
 (via (at 168.5 107.5) (size 0.6) (drill 0.3) (layers "F.Cu" "B.Cu") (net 12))
 (segment (start 109.641 87.359) (end 135.339 87.359) (width 0.2) (layer "F.Cu") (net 6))
 (segment (start 135.339 87.359) (end 137.38 89.4) (width 0.2) (layer "F.Cu") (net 6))
 (segment (start 144.95 93.45) (end 140.9 89.4) (width 0.2) (layer "F.Cu") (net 6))
 (segment (start 96.101 86.248943) (end 96.101 85.751057) (width 0.2) (layer "F.Cu") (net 6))
 (segment (start 146.101 94.551) (end 159.732 80.92) (width 0.2) (layer "F.Cu") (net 6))
 (segment (start 137.38 89.4) (end 137.38 86.12) (width 0.2) (layer "F.Cu") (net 6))
 (segment (start 96.101 85.751057) (end 95.448943 85.099) (width 0.2) (layer "F.Cu") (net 6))
 (segment (start 95.359 87.359) (end 106.656049 87.359) (width 0.2) (layer "F.Cu") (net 6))
 (segment (start 163 80.92) (end 163 74.5) (width 0.2) (layer "F.Cu") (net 6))
 (segment (start 94.601 86.601) (end 95.748943 86.601) (width 0.2) (layer "F.Cu") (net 6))
 (segment (start 107.5 88.202951) (end 107.5 89.5) (width 0.2) (layer "F.Cu") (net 6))
 (segment (start 94.5 86.5) (end 95.359 87.359) (width 0.2) (layer "F.Cu") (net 6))
 (segment (start 155.4 115) (end 154.59 114.19) (width 0.2) (layer "F.Cu") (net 6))
 (segment (start 106.656049 87.359) (end 107.5 88.202951) (width 0.2) (layer "F.Cu") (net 6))
 (segment (start 145 93.45) (end 144.95 93.45) (width 0.2) (layer "F.Cu") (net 6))
 (segment (start 146.101 112.539) (end 146.101 94.551) (width 0.2) (layer "F.Cu") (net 6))
 (segment (start 95.448943 85.099) (end 94.601 85.099) (width 0.2) (layer "F.Cu") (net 6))
 (segment (start 159.732 80.92) (end 163 80.92) (width 0.2) (layer "F.Cu") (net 6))
 (segment (start 140.9 89.4) (end 137.38 89.4) (width 0.2) (layer "F.Cu") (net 6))
 (segment (start 146.101 94.551) (end 145 93.45) (width 0.2) (layer "F.Cu") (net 6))
 (segment (start 94.601 85.099) (end 94.5 85.2) (width 0.2) (layer "F.Cu") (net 6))
 (segment (start 107.5 89.5) (end 106 91) (width 0.2) (layer "F.Cu") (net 6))
 (segment (start 107.5 89.5) (end 109.641 87.359) (width 0.2) (layer "F.Cu") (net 6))
 (segment (start 137.38 86.12) (end 137.5 86) (width 0.2) (layer "F.Cu") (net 6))
 (segment (start 144.45 114.19) (end 146.101 112.539) (width 0.2) (layer "F.Cu") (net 6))
 (segment (start 95.748943 86.601) (end 96.101 86.248943) (width 0.2) (layer "F.Cu") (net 6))
 (segment (start 94.5 86.5) (end 94.601 86.601) (width 0.2) (layer "F.Cu") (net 6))
 (segment (start 154.59 114.19) (end 144.45 114.19) (width 0.2) (layer "F.Cu") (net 6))
 (via (at 91.5 67.5) (size 0.6) (drill 0.3) (layers "F.Cu" "B.Cu") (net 6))
 (via (at 96 82.5) (size 0.6) (drill 0.3) (layers "F.Cu" "B.Cu") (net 6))
 (segment (start 167.5 117.5) (end 167.5 84.5) (width 0.2) (layer "F.Cu") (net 7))
 (segment (start 139.5 116.73) (end 139.846968 116.73) (width 0.2) (layer "F.Cu") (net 7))
 (segment (start 139.846968 116.73) (end 142.616968 119.5) (width 0.2) (layer "F.Cu") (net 7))
 (segment (start 165.5 119.5) (end 167.5 117.5) (width 0.2) (layer "F.Cu") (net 7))
 (segment (start 166.46 83.46) (end 163 83.46) (width 0.2) (layer "F.Cu") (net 7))
 (segment (start 167.5 84.5) (end 166.46 83.46) (width 0.2) (layer "F.Cu") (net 7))
 (segment (start 142.616968 119.5) (end 165.5 119.5) (width 0.2) (layer "F.Cu") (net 7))
 (segment (start 163.47676 70.571) (end 162.52324 70.571) (width 0.2) (layer "F.Cu") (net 4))
 (segment (start 90.998 72.435661) (end 90.998 99.652008) (width 0.2) (layer "F.Cu") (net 4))
 (segment (start 129.516049 79.739) (end 140.986049 68.269) (width 0.2) (layer "F.Cu") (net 4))
 (segment (start 92.9 82.1) (end 94.16 80.84) (width 0.2) (layer "F.Cu") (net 4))
 (segment (start 106 80.84) (end 105.304339 80.84) (width 0.2) (layer "F.Cu") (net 4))
 (segment (start 92.9 84.55) (end 92.9 82.1) (width 0.2) (layer "F.Cu") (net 4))
 (segment (start 101.225339 74.659) (end 123.123951 74.659) (width 0.2) (layer "F.Cu") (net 4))
 (segment (start 162.52324 70.571) (end 145 88.09424) (width 0.2) (layer "F.Cu") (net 4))
 (segment (start 94.16 80.84) (end 106 80.84) (width 0.2) (layer "F.Cu") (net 4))
 (segment (start 111.010942 114.449) (end 117.959942 107.5) (width 0.2) (layer "F.Cu") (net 4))
 (segment (start 95.435339 68.869) (end 101.225339 74.659) (width 0.2) (layer "F.Cu") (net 4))
 (segment (start 105.794992 114.449) (end 111.010942 114.449) (width 0.2) (layer "F.Cu") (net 4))
 (segment (start 93.949 69.484661) (end 94.564661 68.869) (width 0.2) (layer "F.Cu") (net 4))
 (segment (start 94.564661 68.869) (end 95.435339 68.869) (width 0.2) (layer "F.Cu") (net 4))
 (segment (start 164.151 68.94324) (end 164.151 69.89676) (width 0.2) (layer "F.Cu") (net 4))
 (segment (start 93.949 70.355339) (end 93.949 69.484661) (width 0.2) (layer "F.Cu") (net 4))
 (segment (start 105.304339 80.84) (end 95.435339 70.971) (width 0.2) (layer "F.Cu") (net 4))
 (segment (start 123.123951 74.659) (end 128.203951 79.739) (width 0.2) (layer "F.Cu") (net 4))
 (segment (start 94.564661 70.971) (end 93.949 70.355339) (width 0.2) (layer "F.Cu") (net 4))
 (segment (start 140.986049 68.269) (end 163.47676 68.269) (width 0.2) (layer "F.Cu") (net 4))
 (segment (start 145 88.09424) (end 145 89.4) (width 0.2) (layer "F.Cu") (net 4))
 (segment (start 164.151 69.89676) (end 163.47676 70.571) (width 0.2) (layer "F.Cu") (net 4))
 (segment (start 95.435339 70.971) (end 94.564661 70.971) (width 0.2) (layer "F.Cu") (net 4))
 (segment (start 128.203951 79.739) (end 129.516049 79.739) (width 0.2) (layer "F.Cu") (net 4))
 (segment (start 90.998 99.652008) (end 105.794992 114.449) (width 0.2) (layer "F.Cu") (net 4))
 (segment (start 94.564661 68.869) (end 90.998 72.435661) (width 0.2) (layer "F.Cu") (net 4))
 (segment (start 163.47676 68.269) (end 164.151 68.94324) (width 0.2) (layer "F.Cu") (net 4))
 (via (at 152.5 89.5) (size 0.6) (drill 0.3) (layers "F.Cu" "B.Cu") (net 4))
 (via (at 139.5 107.5) (size 0.6) (drill 0.3) (layers "F.Cu" "B.Cu") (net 4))
 (via (at 150 89.5) (size 0.6) (drill 0.3) (layers "F.Cu" "B.Cu") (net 4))
 (via (at 125 107.5) (size 0.6) (drill 0.3) (layers "F.Cu" "B.Cu") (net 4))
 (segment (start 104.608164 64.919) (end 162.66676 64.919) (width 0.2) (layer "F.Cu") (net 5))
 (segment (start 94.5 82.5) (end 95.5 81.5) (width 0.2) (layer "F.Cu") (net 5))
 (segment (start 104.902951 81.5) (end 106 82.597049) (width 0.2) (layer "F.Cu") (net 5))
 (segment (start 103.5 66.027164) (end 104.608164 64.919) (width 0.2) (layer "F.Cu") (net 5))
 (segment (start 106 82.597049) (end 106 83.38) (width 0.2) (layer "F.Cu") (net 5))
 (segment (start 94.5 84.55) (end 94.5 82.5) (width 0.2) (layer "F.Cu") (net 5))
 (segment (start 162.66676 64.919) (end 168.5 70.75224) (width 0.2) (layer "F.Cu") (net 5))
 (segment (start 168.5 70.75224) (end 168.5 102) (width 0.2) (layer "F.Cu") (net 5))
 (segment (start 103.5 67) (end 103.5 66.027164) (width 0.2) (layer "F.Cu") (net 5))
 (segment (start 95.5 81.5) (end 104.902951 81.5) (width 0.2) (layer "F.Cu") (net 5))
 (via (at 104 83.5) (size 0.6) (drill 0.3) (layers "F.Cu" "B.Cu") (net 5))
 (via (at 163 99.5) (size 0.6) (drill 0.3) (layers "F.Cu" "B.Cu") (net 5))
 (via (at 168.5 102) (size 0.6) (drill 0.3) (layers "F.Cu" "B.Cu") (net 5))
 (via (at 103.5 67) (size 0.6) (drill 0.3) (layers "F.Cu" "B.Cu") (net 5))
 (segment (start 140 70) (end 143 70) (width 0.2) (layer "F.Cu") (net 15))
 (segment (start 128.86 80.84) (end 129.16 80.84) (width 0.2) (layer "F.Cu") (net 15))
 (segment (start 143.58 69.42) (end 163 69.42) (width 0.2) (layer "F.Cu") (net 15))
 (segment (start 143 70) (end 143.58 69.42) (width 0.2) (layer "F.Cu") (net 15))
 (segment (start 129.16 80.84) (end 140 70) (width 0.2) (layer "F.Cu") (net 15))
 (segment (start 128.86 77.64) (end 128.86 78.3) (width 0.2) (layer "F.Cu") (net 16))
 (segment (start 163 66.88) (end 139.62 66.88) (width 0.2) (layer "F.Cu") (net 16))
 (segment (start 139.62 66.88) (end 128.86 77.64) (width 0.2) (layer "F.Cu") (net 16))
 (segment (start 136.941 81.941) (end 127.941 81.941) (width 0.2) (layer "F.Cu") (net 10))
 (segment (start 121.76 75.76) (end 106 75.76) (width 0.2) (layer "F.Cu") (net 10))
 (segment (start 137.5 82.5) (end 136.941 81.941) (width 0.2) (layer "F.Cu") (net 10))
 (segment (start 127.941 81.941) (end 121.76 75.76) (width 0.2) (layer "F.Cu") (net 10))
 (via (at 137.5 80) (size 0.6) (drill 0.3) (layers "F.Cu" "B.Cu") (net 10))
 (via (at 141.5 101.5) (size 0.6) (drill 0.3) (layers "F.Cu" "B.Cu") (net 10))
 (via (at 141.5 80) (size 0.6) (drill 0.3) (layers "F.Cu" "B.Cu") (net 10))
 (via (at 152.5 101.5) (size 0.6) (drill 0.3) (layers "F.Cu" "B.Cu") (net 10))
 (segment (start 143.12 84) (end 145.12 86) (width 0.2) (layer "F.Cu") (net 13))
 (segment (start 119.801 76.861) (end 128.86 85.92) (width 0.2) (layer "F.Cu") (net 13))
 (segment (start 128.86 85.92) (end 130.78 84) (width 0.2) (layer "F.Cu") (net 13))
 (segment (start 130.78 84) (end 143.12 84) (width 0.2) (layer "F.Cu") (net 13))
 (segment (start 101.941 76.861) (end 119.801 76.861) (width 0.2) (layer "F.Cu") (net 13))
 (segment (start 95 69.92) (end 101.941 76.861) (width 0.2) (layer "F.Cu") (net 13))
 (segment (start 139.846968 115.46) (end 145 110.306968) (width 0.2) (layer "F.Cu") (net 8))
 (segment (start 145 97.5) (end 144.5 97.5) (width 0.2) (layer "F.Cu") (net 8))
 (segment (start 139.5 115.46) (end 139.846968 115.46) (width 0.2) (layer "F.Cu") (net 8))
 (segment (start 140.45 93.45) (end 137.38 93.45) (width 0.2) (layer "F.Cu") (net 8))
 (segment (start 145 110.306968) (end 145 97.5) (width 0.2) (layer "F.Cu") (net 8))
 (segment (start 144.5 97.5) (end 140.45 93.45) (width 0.2) (layer "F.Cu") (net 8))
 (segment (start 93.949 86.976) (end 95.433 88.46) (width 0.2) (layer "F.Cu") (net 2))
 (segment (start 93.949 86) (end 93.949 86.976) (width 0.2) (layer "F.Cu") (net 2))
 (segment (start 92.9 85.85) (end 93.799 85.85) (width 0.2) (layer "F.Cu") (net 2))
 (segment (start 93.799 85.85) (end 93.949 86) (width 0.2) (layer "F.Cu") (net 2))
 (segment (start 95.433 88.46) (end 106 88.46) (width 0.2) (layer "F.Cu") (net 2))
 (via (at 92 85) (size 0.6) (drill 0.3) (layers "F.Cu" "B.Cu") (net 3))
 (via (at 97 83.5) (size 0.6) (drill 0.3) (layers "F.Cu" "B.Cu") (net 3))
 (via (at 97 85.5) (size 0.6) (drill 0.3) (layers "F.Cu" "B.Cu") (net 3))
 (via (at 92 83.5) (size 0.6) (drill 0.3) (layers "F.Cu" "B.Cu") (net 3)))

